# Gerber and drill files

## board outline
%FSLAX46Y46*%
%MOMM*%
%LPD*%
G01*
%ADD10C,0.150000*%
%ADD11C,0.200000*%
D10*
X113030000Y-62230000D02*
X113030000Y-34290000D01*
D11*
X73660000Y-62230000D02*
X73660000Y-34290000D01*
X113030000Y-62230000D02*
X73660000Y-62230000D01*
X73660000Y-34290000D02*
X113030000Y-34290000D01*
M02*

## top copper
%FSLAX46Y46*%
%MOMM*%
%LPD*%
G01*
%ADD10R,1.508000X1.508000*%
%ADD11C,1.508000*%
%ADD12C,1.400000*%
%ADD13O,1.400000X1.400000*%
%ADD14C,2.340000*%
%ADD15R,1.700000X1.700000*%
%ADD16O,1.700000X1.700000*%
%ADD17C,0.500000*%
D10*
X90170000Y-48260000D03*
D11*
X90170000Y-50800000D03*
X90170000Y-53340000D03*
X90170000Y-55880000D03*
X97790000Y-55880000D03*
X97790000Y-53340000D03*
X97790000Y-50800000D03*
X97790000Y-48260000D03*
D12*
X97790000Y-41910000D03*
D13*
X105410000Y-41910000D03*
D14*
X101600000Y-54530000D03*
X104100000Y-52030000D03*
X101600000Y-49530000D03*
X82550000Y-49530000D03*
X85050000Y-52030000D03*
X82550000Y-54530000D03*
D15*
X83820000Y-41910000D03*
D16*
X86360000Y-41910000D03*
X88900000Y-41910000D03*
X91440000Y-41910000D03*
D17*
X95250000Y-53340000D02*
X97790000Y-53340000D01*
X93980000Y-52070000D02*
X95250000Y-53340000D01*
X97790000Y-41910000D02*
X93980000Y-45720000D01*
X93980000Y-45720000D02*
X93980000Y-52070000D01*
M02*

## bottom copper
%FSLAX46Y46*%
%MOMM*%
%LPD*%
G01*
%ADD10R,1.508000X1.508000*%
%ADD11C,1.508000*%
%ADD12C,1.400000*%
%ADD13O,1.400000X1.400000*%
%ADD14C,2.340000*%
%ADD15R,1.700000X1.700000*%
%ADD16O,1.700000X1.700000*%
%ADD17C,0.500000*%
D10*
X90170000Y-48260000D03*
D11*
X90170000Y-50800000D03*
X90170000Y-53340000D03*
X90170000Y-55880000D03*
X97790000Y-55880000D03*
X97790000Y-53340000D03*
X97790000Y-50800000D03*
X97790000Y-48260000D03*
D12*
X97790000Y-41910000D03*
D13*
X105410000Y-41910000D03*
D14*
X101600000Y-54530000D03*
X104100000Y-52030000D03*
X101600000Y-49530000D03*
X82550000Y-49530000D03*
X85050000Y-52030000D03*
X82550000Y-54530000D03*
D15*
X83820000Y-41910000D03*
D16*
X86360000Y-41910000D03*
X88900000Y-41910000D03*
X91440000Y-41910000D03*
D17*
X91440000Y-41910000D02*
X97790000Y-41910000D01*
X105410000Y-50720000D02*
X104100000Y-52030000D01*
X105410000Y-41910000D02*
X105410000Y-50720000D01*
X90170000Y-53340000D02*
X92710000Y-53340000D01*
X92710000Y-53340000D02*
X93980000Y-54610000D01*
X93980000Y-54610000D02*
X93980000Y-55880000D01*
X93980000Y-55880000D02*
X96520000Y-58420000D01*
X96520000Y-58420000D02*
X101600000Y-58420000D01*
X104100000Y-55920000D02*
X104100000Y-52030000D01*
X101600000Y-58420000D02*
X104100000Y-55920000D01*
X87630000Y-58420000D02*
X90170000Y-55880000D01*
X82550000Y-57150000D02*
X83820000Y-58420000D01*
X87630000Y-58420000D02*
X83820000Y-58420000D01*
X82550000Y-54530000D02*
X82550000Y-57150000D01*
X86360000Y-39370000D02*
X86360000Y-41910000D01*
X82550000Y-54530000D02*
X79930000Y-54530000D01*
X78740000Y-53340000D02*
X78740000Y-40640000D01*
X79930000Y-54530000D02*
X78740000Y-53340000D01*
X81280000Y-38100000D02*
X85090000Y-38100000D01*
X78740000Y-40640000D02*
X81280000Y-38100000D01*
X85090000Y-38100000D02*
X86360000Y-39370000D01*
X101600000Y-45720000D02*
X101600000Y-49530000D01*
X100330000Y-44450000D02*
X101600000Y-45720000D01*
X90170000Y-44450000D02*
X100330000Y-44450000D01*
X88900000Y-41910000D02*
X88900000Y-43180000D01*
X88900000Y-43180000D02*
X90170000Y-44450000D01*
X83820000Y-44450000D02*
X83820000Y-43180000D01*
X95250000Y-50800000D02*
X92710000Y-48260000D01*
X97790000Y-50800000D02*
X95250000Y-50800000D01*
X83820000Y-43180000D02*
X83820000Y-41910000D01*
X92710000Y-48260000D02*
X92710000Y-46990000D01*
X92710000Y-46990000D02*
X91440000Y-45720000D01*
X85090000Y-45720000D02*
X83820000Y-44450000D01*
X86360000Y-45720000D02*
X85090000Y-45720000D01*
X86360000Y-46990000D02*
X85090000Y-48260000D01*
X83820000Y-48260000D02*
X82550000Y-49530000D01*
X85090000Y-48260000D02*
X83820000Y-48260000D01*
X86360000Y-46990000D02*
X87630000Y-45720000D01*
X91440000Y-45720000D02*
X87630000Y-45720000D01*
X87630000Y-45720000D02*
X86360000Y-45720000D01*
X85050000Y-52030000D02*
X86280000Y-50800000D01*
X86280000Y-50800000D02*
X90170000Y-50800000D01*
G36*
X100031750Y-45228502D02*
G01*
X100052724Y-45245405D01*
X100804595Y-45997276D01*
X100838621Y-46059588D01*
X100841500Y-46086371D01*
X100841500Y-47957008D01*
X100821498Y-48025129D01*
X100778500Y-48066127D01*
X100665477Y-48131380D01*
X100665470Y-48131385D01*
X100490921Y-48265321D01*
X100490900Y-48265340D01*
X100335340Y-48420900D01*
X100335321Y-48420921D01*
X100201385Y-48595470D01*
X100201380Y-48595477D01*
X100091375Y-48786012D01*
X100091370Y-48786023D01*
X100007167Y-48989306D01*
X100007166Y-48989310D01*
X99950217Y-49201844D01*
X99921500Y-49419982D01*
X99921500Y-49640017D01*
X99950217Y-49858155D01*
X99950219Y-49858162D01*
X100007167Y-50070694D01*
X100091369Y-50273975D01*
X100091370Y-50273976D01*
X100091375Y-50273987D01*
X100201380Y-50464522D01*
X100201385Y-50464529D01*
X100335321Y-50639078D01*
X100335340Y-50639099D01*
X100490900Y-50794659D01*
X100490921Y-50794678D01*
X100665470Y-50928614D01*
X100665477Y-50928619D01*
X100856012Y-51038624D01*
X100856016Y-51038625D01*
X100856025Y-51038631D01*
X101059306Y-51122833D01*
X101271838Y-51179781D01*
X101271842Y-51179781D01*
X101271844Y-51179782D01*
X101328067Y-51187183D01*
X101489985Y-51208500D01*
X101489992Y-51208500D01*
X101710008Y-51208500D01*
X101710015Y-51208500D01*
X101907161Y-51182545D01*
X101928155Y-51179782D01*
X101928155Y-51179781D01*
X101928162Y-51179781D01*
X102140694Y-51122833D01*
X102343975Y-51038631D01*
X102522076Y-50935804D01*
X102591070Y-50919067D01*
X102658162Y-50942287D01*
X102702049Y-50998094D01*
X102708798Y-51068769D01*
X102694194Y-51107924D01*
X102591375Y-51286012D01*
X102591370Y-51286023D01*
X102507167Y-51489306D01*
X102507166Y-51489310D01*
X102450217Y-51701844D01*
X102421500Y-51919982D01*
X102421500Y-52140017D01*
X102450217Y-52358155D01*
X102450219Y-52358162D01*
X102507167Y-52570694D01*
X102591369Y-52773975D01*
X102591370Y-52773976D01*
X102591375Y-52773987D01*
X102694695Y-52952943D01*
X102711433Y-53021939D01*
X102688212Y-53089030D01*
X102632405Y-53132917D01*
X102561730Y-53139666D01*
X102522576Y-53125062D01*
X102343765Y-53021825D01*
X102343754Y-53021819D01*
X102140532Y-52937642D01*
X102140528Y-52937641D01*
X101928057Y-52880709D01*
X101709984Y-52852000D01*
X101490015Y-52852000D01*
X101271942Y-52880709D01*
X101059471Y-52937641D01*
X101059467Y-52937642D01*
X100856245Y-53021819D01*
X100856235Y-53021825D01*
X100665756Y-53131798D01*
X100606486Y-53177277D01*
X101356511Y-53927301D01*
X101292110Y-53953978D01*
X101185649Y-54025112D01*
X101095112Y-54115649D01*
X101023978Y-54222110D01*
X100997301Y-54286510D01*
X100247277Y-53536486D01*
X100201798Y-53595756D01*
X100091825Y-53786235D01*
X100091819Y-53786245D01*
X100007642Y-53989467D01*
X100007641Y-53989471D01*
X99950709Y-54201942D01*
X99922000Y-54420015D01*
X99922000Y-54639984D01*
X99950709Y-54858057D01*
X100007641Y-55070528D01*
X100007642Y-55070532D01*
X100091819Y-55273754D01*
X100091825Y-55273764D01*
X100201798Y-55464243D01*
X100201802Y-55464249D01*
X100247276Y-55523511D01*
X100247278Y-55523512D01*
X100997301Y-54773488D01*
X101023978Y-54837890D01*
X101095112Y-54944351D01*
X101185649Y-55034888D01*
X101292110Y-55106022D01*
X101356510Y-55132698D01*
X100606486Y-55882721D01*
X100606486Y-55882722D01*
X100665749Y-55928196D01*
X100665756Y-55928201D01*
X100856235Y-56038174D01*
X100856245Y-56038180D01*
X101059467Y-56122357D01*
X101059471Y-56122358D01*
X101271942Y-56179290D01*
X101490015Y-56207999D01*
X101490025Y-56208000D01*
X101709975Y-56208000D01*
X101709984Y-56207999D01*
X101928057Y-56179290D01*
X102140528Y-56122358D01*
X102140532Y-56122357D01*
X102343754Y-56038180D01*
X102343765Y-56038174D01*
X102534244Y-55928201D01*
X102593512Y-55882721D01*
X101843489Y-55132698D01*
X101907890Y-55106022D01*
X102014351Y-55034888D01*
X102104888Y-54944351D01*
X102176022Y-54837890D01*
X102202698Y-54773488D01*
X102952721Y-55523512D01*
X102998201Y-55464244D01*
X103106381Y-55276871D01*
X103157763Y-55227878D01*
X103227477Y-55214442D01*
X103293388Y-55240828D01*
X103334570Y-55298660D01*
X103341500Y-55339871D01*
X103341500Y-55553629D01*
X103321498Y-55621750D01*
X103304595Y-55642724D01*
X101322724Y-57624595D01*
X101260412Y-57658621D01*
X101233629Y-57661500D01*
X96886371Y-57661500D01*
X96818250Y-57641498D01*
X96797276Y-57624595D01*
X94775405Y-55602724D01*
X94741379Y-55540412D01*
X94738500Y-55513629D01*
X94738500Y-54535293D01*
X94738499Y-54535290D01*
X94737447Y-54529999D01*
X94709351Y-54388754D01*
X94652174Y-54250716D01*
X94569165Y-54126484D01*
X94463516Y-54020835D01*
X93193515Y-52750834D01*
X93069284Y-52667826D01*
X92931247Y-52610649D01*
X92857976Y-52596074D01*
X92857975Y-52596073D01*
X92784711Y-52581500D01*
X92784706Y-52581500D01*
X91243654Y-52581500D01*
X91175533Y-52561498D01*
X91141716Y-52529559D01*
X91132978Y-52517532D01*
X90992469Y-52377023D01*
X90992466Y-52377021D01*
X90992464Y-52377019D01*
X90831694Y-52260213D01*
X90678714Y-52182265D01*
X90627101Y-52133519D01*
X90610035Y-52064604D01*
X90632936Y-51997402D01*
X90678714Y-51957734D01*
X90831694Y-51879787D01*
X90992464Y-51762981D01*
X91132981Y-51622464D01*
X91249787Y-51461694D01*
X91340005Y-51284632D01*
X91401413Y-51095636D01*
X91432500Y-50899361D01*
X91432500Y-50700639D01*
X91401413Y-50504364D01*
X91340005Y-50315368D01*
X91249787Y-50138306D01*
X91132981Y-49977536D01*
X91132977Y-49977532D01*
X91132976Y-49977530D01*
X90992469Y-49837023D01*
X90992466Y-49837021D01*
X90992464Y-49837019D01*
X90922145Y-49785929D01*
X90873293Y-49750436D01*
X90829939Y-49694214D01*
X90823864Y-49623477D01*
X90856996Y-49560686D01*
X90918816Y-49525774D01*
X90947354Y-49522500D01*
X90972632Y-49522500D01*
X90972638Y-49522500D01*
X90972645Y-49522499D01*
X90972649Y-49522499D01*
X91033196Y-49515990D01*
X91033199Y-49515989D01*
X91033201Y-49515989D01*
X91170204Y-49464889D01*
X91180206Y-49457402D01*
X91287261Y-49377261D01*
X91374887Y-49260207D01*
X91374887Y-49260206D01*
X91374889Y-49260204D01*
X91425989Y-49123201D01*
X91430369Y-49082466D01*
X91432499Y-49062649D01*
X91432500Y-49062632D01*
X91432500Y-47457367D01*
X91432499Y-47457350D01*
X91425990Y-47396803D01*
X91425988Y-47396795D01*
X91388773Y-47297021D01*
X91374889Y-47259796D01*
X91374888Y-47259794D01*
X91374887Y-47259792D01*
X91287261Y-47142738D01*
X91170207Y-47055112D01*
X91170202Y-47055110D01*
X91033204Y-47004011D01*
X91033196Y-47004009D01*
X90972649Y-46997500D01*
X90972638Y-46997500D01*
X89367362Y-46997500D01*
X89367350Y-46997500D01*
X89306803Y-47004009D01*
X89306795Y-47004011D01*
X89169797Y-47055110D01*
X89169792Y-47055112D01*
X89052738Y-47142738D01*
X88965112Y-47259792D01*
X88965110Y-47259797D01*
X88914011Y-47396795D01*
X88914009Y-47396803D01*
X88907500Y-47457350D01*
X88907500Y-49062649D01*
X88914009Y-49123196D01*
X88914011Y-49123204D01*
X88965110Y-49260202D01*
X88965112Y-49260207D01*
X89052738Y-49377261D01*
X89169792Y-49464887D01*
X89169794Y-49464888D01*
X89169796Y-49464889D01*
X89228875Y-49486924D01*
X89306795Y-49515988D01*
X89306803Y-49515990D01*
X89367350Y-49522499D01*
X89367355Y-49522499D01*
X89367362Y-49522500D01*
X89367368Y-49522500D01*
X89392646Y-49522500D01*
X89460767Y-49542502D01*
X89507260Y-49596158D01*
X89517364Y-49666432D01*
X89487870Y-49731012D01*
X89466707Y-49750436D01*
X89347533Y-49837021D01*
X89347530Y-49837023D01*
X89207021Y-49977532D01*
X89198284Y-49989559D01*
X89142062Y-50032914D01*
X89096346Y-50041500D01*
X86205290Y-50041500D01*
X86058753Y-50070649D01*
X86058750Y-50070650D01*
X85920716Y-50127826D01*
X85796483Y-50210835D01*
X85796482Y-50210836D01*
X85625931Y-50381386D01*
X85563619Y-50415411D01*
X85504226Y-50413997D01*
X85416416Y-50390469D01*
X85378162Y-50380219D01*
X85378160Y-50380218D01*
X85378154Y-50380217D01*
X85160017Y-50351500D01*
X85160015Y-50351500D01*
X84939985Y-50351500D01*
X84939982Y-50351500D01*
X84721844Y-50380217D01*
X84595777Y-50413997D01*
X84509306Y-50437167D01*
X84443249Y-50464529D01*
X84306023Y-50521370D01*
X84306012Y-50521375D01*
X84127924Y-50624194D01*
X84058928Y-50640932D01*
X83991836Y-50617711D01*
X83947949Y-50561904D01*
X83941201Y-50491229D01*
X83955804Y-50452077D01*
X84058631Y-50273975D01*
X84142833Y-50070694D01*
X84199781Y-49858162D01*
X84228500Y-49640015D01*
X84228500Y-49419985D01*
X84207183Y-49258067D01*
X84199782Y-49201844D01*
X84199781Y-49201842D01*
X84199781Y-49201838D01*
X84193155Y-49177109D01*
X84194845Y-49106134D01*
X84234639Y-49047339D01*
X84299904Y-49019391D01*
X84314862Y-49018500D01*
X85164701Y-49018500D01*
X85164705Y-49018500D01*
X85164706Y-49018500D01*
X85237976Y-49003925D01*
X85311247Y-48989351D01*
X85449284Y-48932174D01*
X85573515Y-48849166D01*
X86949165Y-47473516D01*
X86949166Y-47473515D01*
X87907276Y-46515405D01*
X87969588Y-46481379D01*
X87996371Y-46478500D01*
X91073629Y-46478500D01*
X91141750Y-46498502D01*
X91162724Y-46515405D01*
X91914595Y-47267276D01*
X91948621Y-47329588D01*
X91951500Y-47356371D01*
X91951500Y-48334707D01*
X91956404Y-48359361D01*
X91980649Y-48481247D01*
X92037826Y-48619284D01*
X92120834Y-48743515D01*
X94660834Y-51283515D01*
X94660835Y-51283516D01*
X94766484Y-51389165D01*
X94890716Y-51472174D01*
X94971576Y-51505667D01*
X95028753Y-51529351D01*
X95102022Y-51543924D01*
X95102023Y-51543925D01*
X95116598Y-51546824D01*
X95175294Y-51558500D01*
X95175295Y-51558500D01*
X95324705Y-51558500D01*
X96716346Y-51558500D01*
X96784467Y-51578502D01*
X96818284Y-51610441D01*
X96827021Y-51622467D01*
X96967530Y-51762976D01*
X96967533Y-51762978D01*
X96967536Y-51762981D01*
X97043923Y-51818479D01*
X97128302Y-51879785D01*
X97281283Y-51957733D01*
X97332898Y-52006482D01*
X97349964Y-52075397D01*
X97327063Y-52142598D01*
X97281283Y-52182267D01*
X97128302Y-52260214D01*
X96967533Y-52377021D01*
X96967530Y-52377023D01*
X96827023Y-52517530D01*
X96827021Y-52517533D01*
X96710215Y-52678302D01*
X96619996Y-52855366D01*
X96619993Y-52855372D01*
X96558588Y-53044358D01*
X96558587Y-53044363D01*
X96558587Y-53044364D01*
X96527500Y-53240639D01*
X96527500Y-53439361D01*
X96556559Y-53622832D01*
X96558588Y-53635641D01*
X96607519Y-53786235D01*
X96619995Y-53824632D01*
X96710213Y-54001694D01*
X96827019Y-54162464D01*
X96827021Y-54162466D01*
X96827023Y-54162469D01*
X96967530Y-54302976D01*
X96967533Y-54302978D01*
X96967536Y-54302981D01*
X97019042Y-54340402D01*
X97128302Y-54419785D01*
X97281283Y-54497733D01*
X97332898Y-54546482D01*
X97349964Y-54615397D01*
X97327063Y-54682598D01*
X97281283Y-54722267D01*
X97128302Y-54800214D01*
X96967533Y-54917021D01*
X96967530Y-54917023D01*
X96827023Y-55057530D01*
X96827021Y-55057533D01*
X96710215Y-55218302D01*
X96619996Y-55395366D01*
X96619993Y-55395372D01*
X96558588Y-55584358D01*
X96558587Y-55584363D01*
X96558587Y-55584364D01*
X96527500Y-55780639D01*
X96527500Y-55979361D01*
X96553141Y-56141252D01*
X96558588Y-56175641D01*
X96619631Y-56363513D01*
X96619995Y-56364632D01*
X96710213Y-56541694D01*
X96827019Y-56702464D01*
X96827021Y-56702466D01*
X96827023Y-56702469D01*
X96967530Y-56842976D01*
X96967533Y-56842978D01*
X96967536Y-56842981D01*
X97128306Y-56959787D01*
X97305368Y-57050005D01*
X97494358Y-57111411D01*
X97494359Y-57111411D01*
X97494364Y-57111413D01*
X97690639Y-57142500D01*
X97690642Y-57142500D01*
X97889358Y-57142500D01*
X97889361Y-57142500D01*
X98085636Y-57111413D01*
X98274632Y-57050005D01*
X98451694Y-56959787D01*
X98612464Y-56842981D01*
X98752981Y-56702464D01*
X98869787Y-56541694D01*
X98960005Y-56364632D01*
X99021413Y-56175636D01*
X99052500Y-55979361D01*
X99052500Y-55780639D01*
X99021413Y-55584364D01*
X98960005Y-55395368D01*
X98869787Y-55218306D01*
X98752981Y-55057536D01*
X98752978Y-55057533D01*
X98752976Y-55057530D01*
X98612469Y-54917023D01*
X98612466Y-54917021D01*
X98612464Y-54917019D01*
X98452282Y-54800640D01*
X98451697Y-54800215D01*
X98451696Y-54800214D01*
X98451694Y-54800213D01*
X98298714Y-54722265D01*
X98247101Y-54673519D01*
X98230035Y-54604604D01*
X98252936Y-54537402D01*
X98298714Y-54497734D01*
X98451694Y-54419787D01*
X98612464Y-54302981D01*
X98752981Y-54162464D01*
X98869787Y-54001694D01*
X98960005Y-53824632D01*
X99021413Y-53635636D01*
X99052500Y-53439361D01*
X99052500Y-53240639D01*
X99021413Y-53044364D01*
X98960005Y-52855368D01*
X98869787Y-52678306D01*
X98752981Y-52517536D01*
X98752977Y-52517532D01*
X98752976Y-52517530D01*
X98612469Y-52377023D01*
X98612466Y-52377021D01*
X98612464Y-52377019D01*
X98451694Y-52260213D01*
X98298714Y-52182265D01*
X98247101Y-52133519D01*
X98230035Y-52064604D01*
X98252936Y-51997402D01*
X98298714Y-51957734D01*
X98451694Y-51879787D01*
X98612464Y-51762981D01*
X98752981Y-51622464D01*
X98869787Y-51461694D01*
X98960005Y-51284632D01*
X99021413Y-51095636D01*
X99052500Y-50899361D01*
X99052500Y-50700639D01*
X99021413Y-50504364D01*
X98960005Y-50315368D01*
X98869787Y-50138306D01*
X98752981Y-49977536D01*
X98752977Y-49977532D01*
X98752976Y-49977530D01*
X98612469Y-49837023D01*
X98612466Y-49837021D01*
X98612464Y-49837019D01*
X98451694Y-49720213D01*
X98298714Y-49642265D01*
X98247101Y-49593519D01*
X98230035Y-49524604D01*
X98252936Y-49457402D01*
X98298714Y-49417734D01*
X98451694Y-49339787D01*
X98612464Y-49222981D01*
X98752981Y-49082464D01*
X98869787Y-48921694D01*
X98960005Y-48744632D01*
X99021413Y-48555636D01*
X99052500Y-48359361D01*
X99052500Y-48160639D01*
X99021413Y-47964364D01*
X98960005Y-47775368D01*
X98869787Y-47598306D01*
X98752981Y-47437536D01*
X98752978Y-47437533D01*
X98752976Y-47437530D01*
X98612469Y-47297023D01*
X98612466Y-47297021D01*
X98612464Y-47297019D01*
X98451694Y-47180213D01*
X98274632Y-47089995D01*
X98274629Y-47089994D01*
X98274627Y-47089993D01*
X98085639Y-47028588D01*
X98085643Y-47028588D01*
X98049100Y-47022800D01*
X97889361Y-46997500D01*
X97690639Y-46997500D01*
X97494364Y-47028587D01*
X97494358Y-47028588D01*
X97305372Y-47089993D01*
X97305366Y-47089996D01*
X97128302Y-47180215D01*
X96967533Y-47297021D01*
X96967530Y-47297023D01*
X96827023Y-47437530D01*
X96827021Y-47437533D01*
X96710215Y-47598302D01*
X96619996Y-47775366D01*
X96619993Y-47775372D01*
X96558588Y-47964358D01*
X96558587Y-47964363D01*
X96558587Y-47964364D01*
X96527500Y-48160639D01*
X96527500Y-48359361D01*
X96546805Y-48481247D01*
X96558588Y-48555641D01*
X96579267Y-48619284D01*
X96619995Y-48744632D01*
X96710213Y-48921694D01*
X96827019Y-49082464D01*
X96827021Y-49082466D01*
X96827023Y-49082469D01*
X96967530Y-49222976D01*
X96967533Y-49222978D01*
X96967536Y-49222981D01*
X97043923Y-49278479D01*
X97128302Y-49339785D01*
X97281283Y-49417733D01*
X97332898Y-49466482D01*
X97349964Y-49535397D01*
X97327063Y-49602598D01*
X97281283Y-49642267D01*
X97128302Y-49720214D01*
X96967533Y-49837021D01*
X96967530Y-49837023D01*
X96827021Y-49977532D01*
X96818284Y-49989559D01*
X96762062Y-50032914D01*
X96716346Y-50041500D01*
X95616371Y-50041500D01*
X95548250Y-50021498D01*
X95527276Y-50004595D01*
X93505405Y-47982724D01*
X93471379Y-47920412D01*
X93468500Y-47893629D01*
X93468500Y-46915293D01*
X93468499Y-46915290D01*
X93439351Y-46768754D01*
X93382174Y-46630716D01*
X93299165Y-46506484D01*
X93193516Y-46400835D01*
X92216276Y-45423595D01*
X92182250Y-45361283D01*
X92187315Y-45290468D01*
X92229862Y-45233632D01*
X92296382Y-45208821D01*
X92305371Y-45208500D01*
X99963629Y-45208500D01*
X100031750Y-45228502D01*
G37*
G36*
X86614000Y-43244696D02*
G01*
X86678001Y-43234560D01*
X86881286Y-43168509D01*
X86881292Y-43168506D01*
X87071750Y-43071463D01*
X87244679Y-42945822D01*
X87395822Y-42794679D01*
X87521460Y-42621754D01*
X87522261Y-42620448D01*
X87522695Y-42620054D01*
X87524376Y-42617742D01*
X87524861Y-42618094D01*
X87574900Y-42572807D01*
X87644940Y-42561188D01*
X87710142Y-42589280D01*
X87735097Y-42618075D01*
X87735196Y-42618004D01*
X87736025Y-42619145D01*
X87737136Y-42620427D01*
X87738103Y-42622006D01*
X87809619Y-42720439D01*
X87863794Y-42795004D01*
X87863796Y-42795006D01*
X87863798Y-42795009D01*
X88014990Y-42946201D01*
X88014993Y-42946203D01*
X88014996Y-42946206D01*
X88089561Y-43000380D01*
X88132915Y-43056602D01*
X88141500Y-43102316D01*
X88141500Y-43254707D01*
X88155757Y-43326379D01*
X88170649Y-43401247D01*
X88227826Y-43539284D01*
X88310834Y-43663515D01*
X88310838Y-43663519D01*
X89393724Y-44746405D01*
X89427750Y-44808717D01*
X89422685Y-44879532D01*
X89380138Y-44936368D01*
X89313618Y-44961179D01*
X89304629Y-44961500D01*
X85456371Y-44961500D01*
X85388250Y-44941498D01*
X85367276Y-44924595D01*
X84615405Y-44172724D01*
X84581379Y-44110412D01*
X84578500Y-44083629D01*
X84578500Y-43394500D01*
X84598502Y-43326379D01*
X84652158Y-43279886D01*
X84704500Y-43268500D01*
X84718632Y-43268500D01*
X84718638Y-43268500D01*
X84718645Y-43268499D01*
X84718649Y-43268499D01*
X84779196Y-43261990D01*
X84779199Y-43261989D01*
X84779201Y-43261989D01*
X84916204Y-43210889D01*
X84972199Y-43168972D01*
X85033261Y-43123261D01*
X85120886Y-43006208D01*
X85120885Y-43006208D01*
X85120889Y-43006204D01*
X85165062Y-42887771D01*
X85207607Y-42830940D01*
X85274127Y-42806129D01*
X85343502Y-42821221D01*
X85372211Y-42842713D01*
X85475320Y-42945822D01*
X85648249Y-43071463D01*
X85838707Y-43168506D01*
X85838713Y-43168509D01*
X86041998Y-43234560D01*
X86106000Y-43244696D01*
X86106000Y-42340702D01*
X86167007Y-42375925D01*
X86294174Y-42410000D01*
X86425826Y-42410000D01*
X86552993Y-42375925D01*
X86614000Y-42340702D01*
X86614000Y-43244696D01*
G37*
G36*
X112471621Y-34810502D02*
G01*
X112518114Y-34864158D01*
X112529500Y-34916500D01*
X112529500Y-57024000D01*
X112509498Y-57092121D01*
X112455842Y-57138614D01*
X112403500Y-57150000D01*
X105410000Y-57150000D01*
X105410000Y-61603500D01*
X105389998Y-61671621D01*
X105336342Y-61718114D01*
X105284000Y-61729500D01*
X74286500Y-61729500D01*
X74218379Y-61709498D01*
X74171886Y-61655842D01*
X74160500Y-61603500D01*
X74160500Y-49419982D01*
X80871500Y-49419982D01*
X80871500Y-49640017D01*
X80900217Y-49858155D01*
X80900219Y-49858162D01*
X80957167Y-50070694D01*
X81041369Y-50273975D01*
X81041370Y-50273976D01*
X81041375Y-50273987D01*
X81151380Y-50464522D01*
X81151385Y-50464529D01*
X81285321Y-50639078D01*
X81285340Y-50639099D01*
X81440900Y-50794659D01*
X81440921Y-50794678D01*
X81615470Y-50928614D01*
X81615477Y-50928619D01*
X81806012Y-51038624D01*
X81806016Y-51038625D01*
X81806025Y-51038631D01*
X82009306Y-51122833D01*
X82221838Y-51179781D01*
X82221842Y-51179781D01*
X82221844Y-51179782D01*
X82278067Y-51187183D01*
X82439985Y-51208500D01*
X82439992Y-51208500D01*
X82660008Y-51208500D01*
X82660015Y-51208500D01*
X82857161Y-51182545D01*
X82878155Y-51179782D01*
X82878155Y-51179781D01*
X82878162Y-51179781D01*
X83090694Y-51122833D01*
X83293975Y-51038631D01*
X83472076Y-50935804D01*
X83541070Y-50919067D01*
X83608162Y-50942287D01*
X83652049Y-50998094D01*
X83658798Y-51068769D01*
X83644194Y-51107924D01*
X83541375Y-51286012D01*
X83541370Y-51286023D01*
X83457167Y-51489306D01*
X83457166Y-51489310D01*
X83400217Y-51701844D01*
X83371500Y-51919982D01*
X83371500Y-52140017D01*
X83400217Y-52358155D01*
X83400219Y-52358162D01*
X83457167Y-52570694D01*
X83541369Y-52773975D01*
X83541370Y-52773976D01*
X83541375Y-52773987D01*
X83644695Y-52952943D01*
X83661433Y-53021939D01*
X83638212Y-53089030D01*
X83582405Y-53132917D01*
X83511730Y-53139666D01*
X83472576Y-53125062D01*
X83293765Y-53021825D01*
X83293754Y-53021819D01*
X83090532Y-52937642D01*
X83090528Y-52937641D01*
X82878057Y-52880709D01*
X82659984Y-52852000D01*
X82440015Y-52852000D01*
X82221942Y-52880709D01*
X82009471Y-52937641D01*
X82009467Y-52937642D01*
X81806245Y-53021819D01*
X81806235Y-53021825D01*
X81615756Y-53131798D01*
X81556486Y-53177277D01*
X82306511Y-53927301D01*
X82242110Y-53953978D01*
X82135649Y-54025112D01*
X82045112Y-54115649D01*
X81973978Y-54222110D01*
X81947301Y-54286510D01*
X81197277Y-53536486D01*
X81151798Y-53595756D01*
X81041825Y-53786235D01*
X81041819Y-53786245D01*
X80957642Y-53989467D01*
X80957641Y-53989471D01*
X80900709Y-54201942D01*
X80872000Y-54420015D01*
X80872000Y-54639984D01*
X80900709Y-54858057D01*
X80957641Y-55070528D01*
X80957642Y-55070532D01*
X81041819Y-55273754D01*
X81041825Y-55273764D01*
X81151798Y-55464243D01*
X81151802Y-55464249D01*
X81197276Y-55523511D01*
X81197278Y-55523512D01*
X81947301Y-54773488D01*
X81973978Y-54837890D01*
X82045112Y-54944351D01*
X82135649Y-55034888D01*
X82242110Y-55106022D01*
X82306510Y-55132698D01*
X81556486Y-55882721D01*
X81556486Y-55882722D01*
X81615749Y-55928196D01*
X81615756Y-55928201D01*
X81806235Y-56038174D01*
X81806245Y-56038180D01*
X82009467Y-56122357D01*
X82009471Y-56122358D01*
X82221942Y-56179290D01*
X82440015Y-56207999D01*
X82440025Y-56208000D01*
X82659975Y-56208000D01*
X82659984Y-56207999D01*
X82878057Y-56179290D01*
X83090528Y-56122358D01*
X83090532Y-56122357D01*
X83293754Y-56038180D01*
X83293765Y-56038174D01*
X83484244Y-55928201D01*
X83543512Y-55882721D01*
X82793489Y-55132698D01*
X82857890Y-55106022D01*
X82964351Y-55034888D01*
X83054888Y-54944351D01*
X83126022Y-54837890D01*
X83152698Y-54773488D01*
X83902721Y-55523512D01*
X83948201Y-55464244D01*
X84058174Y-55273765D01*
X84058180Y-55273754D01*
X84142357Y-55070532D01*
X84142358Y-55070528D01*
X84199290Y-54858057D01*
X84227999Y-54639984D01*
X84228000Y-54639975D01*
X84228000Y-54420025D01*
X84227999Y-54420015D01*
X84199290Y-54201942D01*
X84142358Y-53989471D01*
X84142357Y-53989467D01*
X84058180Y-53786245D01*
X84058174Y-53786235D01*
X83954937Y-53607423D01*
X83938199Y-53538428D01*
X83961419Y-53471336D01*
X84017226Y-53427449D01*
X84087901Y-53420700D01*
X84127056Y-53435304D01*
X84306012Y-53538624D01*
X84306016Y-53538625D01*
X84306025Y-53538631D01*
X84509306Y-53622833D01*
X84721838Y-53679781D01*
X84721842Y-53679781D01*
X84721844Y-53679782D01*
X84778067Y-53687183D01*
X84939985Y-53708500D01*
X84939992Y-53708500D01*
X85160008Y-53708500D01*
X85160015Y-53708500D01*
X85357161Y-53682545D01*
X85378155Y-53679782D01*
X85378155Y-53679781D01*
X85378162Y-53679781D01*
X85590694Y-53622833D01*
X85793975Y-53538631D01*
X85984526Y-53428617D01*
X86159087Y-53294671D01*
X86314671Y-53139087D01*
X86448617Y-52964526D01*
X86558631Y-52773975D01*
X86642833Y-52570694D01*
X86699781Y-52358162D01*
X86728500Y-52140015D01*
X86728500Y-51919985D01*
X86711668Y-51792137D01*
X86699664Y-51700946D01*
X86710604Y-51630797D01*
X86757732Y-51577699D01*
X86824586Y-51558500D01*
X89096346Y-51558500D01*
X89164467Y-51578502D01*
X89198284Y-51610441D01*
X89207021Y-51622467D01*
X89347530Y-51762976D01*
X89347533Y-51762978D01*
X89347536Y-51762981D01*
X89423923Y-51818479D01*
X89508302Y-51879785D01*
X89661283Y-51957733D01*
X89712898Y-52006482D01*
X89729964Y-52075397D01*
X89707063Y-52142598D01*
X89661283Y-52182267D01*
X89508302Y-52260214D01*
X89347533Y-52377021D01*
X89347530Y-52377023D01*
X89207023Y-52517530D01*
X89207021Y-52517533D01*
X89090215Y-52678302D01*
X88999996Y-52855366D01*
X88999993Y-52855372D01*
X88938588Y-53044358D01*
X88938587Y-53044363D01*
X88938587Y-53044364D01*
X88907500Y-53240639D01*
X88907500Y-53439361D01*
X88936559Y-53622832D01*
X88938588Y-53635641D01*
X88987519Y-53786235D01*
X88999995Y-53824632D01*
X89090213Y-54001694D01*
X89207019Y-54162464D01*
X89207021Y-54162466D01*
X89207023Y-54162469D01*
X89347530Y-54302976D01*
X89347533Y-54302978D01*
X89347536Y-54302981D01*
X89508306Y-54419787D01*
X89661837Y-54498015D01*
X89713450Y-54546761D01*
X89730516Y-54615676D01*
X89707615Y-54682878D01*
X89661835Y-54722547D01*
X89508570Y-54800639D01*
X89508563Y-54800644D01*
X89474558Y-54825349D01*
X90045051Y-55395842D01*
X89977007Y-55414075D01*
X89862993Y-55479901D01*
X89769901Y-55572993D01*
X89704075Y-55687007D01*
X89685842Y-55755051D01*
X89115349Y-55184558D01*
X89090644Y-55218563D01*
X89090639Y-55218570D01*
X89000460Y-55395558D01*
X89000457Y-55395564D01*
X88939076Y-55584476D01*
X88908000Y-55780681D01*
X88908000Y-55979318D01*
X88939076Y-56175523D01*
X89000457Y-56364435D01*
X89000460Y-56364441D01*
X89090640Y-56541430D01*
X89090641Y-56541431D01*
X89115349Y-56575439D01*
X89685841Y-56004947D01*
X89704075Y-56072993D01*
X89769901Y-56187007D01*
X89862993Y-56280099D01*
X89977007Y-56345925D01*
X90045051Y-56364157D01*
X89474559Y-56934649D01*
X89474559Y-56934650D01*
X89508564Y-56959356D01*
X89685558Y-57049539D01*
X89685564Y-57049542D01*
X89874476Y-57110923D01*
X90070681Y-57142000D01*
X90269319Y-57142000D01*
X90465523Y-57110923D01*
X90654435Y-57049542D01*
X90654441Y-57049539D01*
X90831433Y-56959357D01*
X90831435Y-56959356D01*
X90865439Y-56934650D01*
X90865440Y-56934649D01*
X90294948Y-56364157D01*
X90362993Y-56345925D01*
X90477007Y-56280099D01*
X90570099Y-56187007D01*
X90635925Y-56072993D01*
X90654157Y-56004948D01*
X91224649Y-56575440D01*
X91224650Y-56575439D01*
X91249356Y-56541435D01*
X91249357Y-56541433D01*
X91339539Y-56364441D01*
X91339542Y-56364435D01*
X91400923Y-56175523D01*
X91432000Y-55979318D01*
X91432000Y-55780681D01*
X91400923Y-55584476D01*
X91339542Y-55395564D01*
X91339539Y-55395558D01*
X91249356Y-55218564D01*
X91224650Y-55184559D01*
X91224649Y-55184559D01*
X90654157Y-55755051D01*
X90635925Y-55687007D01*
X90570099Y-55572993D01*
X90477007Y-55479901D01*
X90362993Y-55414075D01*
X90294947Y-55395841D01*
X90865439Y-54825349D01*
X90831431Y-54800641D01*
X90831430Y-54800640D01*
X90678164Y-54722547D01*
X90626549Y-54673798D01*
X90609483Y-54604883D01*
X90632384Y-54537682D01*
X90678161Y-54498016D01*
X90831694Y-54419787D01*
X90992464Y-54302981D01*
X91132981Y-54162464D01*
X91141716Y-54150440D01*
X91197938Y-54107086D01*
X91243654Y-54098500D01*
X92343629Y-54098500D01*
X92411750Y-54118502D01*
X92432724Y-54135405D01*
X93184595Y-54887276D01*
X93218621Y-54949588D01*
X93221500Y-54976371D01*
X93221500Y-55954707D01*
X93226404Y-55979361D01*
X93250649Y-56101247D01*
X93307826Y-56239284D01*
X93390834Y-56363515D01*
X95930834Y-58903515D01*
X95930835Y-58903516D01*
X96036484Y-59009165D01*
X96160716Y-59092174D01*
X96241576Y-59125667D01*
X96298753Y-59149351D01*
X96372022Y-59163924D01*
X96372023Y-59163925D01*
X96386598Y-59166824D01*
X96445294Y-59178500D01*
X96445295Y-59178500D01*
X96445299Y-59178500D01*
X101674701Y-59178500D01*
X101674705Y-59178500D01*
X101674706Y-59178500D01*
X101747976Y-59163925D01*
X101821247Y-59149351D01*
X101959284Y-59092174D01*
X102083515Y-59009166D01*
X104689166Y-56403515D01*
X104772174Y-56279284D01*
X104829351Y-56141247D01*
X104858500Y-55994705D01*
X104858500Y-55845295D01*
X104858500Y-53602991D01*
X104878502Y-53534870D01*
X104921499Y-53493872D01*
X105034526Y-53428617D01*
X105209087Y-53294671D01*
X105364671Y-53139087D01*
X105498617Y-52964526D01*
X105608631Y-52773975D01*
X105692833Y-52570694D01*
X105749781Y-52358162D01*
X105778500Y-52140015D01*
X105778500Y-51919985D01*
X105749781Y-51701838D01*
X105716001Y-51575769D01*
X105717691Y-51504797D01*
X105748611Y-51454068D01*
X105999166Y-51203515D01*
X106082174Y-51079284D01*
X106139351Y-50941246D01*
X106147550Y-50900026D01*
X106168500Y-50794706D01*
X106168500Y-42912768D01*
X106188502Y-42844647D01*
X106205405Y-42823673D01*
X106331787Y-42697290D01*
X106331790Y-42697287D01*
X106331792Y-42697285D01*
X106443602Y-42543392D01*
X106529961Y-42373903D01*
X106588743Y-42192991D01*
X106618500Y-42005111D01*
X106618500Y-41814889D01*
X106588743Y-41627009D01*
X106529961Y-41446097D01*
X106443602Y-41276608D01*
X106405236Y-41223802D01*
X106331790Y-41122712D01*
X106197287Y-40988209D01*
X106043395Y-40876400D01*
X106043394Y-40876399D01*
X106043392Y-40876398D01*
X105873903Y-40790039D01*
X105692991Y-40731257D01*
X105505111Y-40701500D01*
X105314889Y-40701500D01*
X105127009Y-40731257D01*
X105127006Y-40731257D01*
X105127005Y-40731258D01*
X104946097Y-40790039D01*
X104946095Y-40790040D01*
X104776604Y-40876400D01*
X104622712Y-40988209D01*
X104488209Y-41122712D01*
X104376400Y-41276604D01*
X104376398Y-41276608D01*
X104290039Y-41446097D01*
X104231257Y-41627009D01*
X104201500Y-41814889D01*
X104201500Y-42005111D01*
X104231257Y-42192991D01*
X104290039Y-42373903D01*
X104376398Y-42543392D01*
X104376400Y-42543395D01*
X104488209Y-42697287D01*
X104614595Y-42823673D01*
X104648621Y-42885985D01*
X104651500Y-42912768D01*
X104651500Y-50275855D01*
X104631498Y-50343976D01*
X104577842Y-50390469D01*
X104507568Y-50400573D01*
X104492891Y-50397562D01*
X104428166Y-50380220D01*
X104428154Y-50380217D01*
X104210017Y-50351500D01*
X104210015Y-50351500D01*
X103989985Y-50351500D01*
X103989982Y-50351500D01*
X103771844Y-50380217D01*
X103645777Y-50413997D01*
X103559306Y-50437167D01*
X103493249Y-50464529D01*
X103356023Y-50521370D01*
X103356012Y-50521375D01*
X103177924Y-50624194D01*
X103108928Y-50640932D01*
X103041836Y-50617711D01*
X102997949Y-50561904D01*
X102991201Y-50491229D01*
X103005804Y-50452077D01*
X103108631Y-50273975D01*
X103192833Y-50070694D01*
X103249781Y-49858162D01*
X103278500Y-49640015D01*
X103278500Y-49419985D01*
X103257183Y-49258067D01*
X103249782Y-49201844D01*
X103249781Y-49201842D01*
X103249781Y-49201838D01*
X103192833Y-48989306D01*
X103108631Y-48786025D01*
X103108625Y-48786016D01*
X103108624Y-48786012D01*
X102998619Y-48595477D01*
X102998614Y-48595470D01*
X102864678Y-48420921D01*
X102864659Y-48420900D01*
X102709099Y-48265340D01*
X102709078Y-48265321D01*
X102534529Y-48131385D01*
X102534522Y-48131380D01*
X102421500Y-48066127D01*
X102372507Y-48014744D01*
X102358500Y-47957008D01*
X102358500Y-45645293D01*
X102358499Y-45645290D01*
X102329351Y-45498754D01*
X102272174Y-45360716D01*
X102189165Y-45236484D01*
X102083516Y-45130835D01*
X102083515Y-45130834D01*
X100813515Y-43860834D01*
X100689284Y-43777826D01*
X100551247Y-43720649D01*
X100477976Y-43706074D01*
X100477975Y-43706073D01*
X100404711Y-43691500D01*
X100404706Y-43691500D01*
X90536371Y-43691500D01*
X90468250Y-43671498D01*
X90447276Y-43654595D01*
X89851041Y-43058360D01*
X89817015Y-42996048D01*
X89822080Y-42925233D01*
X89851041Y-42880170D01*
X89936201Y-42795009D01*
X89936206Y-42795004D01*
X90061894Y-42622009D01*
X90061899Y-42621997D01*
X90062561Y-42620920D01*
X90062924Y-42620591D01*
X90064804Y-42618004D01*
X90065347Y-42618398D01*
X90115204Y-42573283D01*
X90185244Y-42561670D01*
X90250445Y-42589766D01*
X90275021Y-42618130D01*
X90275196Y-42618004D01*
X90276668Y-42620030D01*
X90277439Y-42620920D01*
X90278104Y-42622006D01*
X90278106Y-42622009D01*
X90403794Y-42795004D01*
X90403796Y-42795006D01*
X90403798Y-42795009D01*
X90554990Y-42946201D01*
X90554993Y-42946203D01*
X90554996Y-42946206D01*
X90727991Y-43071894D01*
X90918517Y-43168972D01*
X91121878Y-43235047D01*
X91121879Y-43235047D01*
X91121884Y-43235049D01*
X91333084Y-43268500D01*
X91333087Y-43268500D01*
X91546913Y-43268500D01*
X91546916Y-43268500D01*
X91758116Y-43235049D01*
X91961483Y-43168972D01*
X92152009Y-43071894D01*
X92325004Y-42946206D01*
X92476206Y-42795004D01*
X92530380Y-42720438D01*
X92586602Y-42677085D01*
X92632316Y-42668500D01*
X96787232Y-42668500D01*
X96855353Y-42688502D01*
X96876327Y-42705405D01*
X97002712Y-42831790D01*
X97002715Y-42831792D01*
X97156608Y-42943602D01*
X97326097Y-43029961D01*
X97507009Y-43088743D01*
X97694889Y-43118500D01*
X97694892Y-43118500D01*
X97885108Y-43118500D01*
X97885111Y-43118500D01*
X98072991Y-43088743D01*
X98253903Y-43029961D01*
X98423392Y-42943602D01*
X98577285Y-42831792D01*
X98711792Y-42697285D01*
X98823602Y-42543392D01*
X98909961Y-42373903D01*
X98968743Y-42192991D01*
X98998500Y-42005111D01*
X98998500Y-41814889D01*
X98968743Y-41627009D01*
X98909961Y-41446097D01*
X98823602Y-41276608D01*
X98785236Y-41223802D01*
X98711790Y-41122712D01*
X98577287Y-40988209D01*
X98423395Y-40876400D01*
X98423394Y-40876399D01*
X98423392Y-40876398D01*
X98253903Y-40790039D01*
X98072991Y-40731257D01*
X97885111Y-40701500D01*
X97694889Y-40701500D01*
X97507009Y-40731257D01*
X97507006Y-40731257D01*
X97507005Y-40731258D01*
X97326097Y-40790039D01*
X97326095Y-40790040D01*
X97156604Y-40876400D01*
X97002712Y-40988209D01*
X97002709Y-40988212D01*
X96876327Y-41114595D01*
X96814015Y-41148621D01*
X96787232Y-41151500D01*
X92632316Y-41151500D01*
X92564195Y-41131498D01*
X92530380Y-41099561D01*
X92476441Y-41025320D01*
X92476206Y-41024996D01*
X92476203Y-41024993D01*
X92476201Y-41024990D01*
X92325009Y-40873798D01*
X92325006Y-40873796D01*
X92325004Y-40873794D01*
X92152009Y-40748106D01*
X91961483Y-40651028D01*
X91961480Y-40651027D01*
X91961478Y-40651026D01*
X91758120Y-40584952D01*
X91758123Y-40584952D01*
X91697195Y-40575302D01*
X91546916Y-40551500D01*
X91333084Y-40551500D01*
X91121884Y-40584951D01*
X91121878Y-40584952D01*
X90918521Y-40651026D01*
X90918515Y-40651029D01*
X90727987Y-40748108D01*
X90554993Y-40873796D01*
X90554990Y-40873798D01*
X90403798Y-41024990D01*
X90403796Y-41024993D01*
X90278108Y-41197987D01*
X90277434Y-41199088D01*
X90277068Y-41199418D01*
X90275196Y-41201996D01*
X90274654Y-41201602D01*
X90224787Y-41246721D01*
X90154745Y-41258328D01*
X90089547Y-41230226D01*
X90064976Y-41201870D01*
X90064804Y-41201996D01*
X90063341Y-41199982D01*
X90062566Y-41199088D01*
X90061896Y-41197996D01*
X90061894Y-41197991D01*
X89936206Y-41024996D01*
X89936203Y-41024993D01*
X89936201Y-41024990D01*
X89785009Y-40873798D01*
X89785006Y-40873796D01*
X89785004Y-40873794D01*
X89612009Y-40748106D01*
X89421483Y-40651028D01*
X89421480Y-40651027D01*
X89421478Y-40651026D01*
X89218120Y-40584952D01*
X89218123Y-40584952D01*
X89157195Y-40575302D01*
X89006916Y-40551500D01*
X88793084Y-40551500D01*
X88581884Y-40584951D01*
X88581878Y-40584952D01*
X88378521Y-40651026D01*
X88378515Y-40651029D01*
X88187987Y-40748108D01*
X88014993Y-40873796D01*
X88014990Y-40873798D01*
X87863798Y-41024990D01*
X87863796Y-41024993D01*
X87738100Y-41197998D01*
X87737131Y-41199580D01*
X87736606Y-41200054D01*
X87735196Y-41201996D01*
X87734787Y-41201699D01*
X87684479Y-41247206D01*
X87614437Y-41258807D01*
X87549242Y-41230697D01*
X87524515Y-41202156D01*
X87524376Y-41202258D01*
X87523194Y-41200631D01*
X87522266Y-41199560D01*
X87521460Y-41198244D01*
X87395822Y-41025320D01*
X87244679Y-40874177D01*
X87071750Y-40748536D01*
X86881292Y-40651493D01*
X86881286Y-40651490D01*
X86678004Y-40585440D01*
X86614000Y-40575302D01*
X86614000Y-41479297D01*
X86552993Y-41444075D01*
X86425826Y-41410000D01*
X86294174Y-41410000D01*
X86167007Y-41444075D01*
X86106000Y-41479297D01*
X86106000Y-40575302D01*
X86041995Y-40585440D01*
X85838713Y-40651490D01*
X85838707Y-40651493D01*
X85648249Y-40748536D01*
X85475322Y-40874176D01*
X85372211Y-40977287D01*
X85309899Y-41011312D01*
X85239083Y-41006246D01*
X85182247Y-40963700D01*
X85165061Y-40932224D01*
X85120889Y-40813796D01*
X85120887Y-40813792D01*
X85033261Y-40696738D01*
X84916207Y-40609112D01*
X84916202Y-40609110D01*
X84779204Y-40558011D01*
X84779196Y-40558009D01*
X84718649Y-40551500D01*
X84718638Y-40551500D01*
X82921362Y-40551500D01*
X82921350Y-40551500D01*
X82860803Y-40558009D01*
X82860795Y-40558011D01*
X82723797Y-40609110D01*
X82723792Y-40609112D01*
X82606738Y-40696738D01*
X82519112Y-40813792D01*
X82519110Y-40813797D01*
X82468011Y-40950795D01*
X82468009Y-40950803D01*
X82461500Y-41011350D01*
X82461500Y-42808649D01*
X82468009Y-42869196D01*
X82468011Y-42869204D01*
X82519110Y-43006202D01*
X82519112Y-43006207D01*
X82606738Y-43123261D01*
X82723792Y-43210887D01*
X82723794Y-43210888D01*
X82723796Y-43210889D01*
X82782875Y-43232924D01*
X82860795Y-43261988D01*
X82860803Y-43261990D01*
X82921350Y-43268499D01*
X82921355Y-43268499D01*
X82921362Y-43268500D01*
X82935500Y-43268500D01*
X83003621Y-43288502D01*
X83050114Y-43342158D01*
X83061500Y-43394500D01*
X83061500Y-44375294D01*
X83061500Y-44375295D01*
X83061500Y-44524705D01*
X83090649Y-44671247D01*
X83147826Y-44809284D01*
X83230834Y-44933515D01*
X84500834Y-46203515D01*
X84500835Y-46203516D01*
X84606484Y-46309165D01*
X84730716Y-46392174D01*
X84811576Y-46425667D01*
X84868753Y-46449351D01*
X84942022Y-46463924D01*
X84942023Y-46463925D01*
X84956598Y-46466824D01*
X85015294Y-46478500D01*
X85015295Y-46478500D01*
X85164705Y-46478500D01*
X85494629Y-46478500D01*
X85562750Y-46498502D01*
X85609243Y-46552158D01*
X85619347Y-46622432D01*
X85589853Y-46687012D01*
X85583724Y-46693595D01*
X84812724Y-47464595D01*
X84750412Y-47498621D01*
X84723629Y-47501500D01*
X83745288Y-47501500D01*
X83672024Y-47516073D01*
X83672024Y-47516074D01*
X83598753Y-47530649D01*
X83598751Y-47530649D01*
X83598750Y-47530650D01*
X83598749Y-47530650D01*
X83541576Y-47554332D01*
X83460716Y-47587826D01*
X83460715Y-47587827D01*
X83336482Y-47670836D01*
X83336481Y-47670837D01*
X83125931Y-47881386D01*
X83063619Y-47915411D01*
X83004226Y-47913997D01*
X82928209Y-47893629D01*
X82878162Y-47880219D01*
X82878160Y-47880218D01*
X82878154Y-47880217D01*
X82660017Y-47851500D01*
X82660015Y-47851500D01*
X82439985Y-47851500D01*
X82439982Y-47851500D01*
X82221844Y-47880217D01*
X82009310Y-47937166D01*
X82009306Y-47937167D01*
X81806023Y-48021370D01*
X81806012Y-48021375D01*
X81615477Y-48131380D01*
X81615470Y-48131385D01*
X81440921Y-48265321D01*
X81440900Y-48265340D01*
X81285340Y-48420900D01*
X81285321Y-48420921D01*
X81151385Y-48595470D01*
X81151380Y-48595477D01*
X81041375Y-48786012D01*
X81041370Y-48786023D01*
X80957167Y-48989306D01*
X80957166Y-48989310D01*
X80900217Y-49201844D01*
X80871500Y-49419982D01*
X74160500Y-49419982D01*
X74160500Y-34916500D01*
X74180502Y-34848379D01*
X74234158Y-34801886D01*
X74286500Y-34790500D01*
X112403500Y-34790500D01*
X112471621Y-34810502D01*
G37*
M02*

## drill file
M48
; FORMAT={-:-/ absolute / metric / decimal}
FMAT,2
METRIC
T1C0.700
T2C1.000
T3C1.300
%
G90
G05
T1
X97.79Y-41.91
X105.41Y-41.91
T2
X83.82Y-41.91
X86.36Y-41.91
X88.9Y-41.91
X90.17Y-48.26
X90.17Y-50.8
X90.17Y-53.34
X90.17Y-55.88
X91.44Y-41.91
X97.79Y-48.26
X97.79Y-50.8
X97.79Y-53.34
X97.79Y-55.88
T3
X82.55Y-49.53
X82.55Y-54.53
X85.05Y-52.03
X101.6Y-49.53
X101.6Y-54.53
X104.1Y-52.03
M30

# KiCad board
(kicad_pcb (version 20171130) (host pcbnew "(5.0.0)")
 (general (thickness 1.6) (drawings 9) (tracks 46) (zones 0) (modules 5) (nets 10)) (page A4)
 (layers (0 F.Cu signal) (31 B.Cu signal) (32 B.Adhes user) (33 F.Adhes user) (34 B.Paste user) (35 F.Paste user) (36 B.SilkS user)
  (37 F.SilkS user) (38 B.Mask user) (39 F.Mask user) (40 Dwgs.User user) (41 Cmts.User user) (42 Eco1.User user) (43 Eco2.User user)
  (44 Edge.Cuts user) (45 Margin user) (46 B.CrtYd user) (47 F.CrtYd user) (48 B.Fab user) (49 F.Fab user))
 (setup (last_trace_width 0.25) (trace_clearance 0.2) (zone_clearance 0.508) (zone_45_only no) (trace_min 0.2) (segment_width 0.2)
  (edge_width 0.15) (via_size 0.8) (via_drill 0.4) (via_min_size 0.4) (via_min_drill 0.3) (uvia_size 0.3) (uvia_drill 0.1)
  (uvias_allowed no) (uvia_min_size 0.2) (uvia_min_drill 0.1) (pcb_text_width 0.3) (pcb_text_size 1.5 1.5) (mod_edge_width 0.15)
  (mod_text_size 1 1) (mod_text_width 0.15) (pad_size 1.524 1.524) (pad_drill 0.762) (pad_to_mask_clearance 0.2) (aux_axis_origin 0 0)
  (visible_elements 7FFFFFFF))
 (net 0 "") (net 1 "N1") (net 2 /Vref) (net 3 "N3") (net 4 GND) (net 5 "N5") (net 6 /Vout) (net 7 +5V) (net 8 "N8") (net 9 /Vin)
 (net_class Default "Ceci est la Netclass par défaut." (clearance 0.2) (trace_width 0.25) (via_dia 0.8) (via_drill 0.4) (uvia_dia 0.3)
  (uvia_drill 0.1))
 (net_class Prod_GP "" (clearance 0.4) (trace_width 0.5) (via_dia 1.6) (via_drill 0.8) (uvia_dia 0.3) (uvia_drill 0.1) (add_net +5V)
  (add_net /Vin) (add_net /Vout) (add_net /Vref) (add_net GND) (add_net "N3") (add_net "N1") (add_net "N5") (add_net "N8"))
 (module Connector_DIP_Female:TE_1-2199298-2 (layer F.Cu) (at 93.98 52.07)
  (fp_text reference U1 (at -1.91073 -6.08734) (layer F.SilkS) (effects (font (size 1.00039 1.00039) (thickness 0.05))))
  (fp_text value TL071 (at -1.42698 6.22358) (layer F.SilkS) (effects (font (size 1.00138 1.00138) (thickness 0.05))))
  (pad 1 thru_hole rect (at -3.81 -3.81) (size 1.508 1.508) (drill 1) (layers *.Cu *.Mask) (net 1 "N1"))
  (pad 2 thru_hole circle (at -3.81 -1.27) (size 1.508 1.508) (drill 1) (layers *.Cu *.Mask) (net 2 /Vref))
  (pad 3 thru_hole circle (at -3.81 1.27) (size 1.508 1.508) (drill 1) (layers *.Cu *.Mask) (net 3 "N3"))
  (pad 4 thru_hole circle (at -3.81 3.81) (size 1.508 1.508) (drill 1) (layers *.Cu *.Mask) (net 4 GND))
  (pad 5 thru_hole circle (at 3.81 3.81) (size 1.508 1.508) (drill 1) (layers *.Cu *.Mask) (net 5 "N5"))
  (pad 6 thru_hole circle (at 3.81 1.27) (size 1.508 1.508) (drill 1) (layers *.Cu *.Mask) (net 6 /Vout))
  (pad 7 thru_hole circle (at 3.81 -1.27) (size 1.508 1.508) (drill 1) (layers *.Cu *.Mask) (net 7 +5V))
  (pad 8 thru_hole circle (at 3.81 -3.81) (size 1.508 1.508) (drill 1) (layers *.Cu *.Mask) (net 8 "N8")))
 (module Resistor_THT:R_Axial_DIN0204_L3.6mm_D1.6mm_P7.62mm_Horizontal (layer F.Cu) (at 97.79 41.91)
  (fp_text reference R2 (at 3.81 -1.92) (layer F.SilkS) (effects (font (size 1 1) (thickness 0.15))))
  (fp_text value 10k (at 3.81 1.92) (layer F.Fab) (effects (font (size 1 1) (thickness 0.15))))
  (pad 1 thru_hole circle (at 0 0) (size 1.4 1.4) (drill 0.7) (layers *.Cu *.Mask) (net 6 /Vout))
  (pad 2 thru_hole oval (at 7.62 0) (size 1.4 1.4) (drill 0.7) (layers *.Cu *.Mask) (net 3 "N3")))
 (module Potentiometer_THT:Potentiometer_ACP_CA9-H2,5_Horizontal (layer F.Cu) (at 101.6 49.53)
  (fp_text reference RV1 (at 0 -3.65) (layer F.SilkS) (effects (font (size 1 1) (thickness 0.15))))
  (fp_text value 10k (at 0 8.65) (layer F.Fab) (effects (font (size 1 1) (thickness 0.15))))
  (pad 3 thru_hole circle (at 0 5) (size 2.34 2.34) (drill 1.3) (layers *.Cu *.Mask) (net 4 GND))
  (pad 2 thru_hole circle (at 2.5 2.5) (size 2.34 2.34) (drill 1.3) (layers *.Cu *.Mask) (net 3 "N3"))
  (pad 1 thru_hole circle (at 0 0) (size 2.34 2.34) (drill 1.3) (layers *.Cu *.Mask) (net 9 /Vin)))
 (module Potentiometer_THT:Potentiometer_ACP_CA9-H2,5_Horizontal (layer F.Cu) (at 82.55 49.53)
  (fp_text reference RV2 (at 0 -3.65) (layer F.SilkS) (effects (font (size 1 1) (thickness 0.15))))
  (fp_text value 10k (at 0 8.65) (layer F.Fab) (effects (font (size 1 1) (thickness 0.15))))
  (pad 1 thru_hole circle (at 0 0) (size 2.34 2.34) (drill 1.3) (layers *.Cu *.Mask) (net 7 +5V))
  (pad 2 thru_hole circle (at 2.5 2.5) (size 2.34 2.34) (drill 1.3) (layers *.Cu *.Mask) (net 2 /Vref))
  (pad 3 thru_hole circle (at 0 5) (size 2.34 2.34) (drill 1.3) (layers *.Cu *.Mask) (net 4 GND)))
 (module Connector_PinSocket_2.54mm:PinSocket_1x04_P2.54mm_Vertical (layer F.Cu) (at 83.82 41.91 90)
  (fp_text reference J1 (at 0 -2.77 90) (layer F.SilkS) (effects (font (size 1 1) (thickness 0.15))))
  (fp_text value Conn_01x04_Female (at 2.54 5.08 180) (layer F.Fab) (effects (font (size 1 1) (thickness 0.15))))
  (pad 1 thru_hole rect (at 0 0 90) (size 1.7 1.7) (drill 1) (layers *.Cu *.Mask) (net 7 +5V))
  (pad 2 thru_hole oval (at 0 2.54 90) (size 1.7 1.7) (drill 1) (layers *.Cu *.Mask) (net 4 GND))
  (pad 3 thru_hole oval (at 0 5.08 90) (size 1.7 1.7) (drill 1) (layers *.Cu *.Mask) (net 9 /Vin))
  (pad 4 thru_hole oval (at 0 7.62 90) (size 1.7 1.7) (drill 1) (layers *.Cu *.Mask) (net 6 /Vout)))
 (gr_line (start 113.03 62.23) (end 113.03 34.29) (layer Edge.Cuts) (width 0.15))
 (gr_line (start 73.66 62.23) (end 73.66 34.29) (layer Edge.Cuts) (width 0.2))
 (gr_line (start 113.03 62.23) (end 73.66 62.23) (layer Edge.Cuts) (width 0.2))
 (gr_line (start 73.66 34.29) (end 113.03 34.29) (layer Edge.Cuts) (width 0.2))
 (segment (start 91.44 41.91) (end 97.79 41.91) (width 0.5) (layer B.Cu) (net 6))
 (segment (start 95.25 53.34) (end 97.79 53.34) (width 0.5) (layer F.Cu) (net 6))
 (segment (start 93.98 52.07) (end 95.25 53.34) (width 0.5) (layer F.Cu) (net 6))
 (segment (start 97.79 41.91) (end 93.98 45.72) (width 0.5) (layer F.Cu) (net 6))
 (segment (start 93.98 45.72) (end 93.98 52.07) (width 0.5) (layer F.Cu) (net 6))
 (segment (start 105.41 50.72) (end 104.1 52.03) (width 0.5) (layer B.Cu) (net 3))
 (segment (start 105.41 41.91) (end 105.41 50.72) (width 0.5) (layer B.Cu) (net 3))
 (segment (start 90.17 53.34) (end 92.71 53.34) (width 0.5) (layer B.Cu) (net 3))
 (segment (start 92.71 53.34) (end 93.98 54.61) (width 0.5) (layer B.Cu) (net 3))
 (segment (start 93.98 54.61) (end 93.98 55.88) (width 0.5) (layer B.Cu) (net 3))
 (segment (start 93.98 55.88) (end 96.52 58.42) (width 0.5) (layer B.Cu) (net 3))
 (segment (start 96.52 58.42) (end 101.6 58.42) (width 0.5) (layer B.Cu) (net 3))
 (segment (start 104.1 55.92) (end 104.1 52.03) (width 0.5) (layer B.Cu) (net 3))
 (segment (start 101.6 58.42) (end 104.1 55.92) (width 0.5) (layer B.Cu) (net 3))
 (segment (start 87.63 58.42) (end 90.17 55.88) (width 0.5) (layer B.Cu) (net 4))
 (segment (start 82.55 57.15) (end 83.82 58.42) (width 0.5) (layer B.Cu) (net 4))
 (segment (start 87.63 58.42) (end 83.82 58.42) (width 0.5) (layer B.Cu) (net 4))
 (segment (start 82.55 54.53) (end 82.55 57.15) (width 0.5) (layer B.Cu) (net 4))
 (segment (start 86.36 39.37) (end 86.36 41.91) (width 0.5) (layer B.Cu) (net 4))
 (segment (start 82.55 54.53) (end 79.93 54.53) (width 0.5) (layer B.Cu) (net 4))
 (segment (start 78.74 53.34) (end 78.74 40.64) (width 0.5) (layer B.Cu) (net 4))
 (segment (start 79.93 54.53) (end 78.74 53.34) (width 0.5) (layer B.Cu) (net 4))
 (segment (start 81.28 38.1) (end 85.09 38.1) (width 0.5) (layer B.Cu) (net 4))
 (segment (start 78.74 40.64) (end 81.28 38.1) (width 0.5) (layer B.Cu) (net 4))
 (segment (start 85.09 38.1) (end 86.36 39.37) (width 0.5) (layer B.Cu) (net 4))
 (segment (start 101.6 45.72) (end 101.6 49.53) (width 0.5) (layer B.Cu) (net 9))
 (segment (start 100.33 44.45) (end 101.6 45.72) (width 0.5) (layer B.Cu) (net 9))
 (segment (start 90.17 44.45) (end 100.33 44.45) (width 0.5) (layer B.Cu) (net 9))
 (segment (start 88.9 41.91) (end 88.9 43.18) (width 0.5) (layer B.Cu) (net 9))
 (segment (start 88.9 43.18) (end 90.17 44.45) (width 0.5) (layer B.Cu) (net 9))
 (segment (start 83.82 44.45) (end 83.82 43.18) (width 0.5) (layer B.Cu) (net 7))
 (segment (start 95.25 50.8) (end 92.71 48.26) (width 0.5) (layer B.Cu) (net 7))
 (segment (start 97.79 50.8) (end 95.25 50.8) (width 0.5) (layer B.Cu) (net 7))
 (segment (start 83.82 43.18) (end 83.82 41.91) (width 0.5) (layer B.Cu) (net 7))
 (segment (start 92.71 48.26) (end 92.71 46.99) (width 0.5) (layer B.Cu) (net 7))
 (segment (start 92.71 46.99) (end 91.44 45.72) (width 0.5) (layer B.Cu) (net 7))
 (segment (start 85.09 45.72) (end 83.82 44.45) (width 0.5) (layer B.Cu) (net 7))
 (segment (start 86.36 45.72) (end 85.09 45.72) (width 0.5) (layer B.Cu) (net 7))
 (segment (start 86.36 46.99) (end 85.09 48.26) (width 0.5) (layer B.Cu) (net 7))
 (segment (start 83.82 48.26) (end 82.55 49.53) (width 0.5) (layer B.Cu) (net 7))
 (segment (start 85.09 48.26) (end 83.82 48.26) (width 0.5) (layer B.Cu) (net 7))
 (segment (start 86.36 46.99) (end 87.63 45.72) (width 0.5) (layer B.Cu) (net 7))
 (segment (start 91.44 45.72) (end 87.63 45.72) (width 0.5) (layer B.Cu) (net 7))
 (segment (start 87.63 45.72) (end 86.36 45.72) (width 0.5) (layer B.Cu) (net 7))
 (segment (start 85.05 52.03) (end 86.28 50.8) (width 0.5) (layer B.Cu) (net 2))
 (segment (start 86.28 50.8) (end 90.17 50.8) (width 0.5) (layer B.Cu) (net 2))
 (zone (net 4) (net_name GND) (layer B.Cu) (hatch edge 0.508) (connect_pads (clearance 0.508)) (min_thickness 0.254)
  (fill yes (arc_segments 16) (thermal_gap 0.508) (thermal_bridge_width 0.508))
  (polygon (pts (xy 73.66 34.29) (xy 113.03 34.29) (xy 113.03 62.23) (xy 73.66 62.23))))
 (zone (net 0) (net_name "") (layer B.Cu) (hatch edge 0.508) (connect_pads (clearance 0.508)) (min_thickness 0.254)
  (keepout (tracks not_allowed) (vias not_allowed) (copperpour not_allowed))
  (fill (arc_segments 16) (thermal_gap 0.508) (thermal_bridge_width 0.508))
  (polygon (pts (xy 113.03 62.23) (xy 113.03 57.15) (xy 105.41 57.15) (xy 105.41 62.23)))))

